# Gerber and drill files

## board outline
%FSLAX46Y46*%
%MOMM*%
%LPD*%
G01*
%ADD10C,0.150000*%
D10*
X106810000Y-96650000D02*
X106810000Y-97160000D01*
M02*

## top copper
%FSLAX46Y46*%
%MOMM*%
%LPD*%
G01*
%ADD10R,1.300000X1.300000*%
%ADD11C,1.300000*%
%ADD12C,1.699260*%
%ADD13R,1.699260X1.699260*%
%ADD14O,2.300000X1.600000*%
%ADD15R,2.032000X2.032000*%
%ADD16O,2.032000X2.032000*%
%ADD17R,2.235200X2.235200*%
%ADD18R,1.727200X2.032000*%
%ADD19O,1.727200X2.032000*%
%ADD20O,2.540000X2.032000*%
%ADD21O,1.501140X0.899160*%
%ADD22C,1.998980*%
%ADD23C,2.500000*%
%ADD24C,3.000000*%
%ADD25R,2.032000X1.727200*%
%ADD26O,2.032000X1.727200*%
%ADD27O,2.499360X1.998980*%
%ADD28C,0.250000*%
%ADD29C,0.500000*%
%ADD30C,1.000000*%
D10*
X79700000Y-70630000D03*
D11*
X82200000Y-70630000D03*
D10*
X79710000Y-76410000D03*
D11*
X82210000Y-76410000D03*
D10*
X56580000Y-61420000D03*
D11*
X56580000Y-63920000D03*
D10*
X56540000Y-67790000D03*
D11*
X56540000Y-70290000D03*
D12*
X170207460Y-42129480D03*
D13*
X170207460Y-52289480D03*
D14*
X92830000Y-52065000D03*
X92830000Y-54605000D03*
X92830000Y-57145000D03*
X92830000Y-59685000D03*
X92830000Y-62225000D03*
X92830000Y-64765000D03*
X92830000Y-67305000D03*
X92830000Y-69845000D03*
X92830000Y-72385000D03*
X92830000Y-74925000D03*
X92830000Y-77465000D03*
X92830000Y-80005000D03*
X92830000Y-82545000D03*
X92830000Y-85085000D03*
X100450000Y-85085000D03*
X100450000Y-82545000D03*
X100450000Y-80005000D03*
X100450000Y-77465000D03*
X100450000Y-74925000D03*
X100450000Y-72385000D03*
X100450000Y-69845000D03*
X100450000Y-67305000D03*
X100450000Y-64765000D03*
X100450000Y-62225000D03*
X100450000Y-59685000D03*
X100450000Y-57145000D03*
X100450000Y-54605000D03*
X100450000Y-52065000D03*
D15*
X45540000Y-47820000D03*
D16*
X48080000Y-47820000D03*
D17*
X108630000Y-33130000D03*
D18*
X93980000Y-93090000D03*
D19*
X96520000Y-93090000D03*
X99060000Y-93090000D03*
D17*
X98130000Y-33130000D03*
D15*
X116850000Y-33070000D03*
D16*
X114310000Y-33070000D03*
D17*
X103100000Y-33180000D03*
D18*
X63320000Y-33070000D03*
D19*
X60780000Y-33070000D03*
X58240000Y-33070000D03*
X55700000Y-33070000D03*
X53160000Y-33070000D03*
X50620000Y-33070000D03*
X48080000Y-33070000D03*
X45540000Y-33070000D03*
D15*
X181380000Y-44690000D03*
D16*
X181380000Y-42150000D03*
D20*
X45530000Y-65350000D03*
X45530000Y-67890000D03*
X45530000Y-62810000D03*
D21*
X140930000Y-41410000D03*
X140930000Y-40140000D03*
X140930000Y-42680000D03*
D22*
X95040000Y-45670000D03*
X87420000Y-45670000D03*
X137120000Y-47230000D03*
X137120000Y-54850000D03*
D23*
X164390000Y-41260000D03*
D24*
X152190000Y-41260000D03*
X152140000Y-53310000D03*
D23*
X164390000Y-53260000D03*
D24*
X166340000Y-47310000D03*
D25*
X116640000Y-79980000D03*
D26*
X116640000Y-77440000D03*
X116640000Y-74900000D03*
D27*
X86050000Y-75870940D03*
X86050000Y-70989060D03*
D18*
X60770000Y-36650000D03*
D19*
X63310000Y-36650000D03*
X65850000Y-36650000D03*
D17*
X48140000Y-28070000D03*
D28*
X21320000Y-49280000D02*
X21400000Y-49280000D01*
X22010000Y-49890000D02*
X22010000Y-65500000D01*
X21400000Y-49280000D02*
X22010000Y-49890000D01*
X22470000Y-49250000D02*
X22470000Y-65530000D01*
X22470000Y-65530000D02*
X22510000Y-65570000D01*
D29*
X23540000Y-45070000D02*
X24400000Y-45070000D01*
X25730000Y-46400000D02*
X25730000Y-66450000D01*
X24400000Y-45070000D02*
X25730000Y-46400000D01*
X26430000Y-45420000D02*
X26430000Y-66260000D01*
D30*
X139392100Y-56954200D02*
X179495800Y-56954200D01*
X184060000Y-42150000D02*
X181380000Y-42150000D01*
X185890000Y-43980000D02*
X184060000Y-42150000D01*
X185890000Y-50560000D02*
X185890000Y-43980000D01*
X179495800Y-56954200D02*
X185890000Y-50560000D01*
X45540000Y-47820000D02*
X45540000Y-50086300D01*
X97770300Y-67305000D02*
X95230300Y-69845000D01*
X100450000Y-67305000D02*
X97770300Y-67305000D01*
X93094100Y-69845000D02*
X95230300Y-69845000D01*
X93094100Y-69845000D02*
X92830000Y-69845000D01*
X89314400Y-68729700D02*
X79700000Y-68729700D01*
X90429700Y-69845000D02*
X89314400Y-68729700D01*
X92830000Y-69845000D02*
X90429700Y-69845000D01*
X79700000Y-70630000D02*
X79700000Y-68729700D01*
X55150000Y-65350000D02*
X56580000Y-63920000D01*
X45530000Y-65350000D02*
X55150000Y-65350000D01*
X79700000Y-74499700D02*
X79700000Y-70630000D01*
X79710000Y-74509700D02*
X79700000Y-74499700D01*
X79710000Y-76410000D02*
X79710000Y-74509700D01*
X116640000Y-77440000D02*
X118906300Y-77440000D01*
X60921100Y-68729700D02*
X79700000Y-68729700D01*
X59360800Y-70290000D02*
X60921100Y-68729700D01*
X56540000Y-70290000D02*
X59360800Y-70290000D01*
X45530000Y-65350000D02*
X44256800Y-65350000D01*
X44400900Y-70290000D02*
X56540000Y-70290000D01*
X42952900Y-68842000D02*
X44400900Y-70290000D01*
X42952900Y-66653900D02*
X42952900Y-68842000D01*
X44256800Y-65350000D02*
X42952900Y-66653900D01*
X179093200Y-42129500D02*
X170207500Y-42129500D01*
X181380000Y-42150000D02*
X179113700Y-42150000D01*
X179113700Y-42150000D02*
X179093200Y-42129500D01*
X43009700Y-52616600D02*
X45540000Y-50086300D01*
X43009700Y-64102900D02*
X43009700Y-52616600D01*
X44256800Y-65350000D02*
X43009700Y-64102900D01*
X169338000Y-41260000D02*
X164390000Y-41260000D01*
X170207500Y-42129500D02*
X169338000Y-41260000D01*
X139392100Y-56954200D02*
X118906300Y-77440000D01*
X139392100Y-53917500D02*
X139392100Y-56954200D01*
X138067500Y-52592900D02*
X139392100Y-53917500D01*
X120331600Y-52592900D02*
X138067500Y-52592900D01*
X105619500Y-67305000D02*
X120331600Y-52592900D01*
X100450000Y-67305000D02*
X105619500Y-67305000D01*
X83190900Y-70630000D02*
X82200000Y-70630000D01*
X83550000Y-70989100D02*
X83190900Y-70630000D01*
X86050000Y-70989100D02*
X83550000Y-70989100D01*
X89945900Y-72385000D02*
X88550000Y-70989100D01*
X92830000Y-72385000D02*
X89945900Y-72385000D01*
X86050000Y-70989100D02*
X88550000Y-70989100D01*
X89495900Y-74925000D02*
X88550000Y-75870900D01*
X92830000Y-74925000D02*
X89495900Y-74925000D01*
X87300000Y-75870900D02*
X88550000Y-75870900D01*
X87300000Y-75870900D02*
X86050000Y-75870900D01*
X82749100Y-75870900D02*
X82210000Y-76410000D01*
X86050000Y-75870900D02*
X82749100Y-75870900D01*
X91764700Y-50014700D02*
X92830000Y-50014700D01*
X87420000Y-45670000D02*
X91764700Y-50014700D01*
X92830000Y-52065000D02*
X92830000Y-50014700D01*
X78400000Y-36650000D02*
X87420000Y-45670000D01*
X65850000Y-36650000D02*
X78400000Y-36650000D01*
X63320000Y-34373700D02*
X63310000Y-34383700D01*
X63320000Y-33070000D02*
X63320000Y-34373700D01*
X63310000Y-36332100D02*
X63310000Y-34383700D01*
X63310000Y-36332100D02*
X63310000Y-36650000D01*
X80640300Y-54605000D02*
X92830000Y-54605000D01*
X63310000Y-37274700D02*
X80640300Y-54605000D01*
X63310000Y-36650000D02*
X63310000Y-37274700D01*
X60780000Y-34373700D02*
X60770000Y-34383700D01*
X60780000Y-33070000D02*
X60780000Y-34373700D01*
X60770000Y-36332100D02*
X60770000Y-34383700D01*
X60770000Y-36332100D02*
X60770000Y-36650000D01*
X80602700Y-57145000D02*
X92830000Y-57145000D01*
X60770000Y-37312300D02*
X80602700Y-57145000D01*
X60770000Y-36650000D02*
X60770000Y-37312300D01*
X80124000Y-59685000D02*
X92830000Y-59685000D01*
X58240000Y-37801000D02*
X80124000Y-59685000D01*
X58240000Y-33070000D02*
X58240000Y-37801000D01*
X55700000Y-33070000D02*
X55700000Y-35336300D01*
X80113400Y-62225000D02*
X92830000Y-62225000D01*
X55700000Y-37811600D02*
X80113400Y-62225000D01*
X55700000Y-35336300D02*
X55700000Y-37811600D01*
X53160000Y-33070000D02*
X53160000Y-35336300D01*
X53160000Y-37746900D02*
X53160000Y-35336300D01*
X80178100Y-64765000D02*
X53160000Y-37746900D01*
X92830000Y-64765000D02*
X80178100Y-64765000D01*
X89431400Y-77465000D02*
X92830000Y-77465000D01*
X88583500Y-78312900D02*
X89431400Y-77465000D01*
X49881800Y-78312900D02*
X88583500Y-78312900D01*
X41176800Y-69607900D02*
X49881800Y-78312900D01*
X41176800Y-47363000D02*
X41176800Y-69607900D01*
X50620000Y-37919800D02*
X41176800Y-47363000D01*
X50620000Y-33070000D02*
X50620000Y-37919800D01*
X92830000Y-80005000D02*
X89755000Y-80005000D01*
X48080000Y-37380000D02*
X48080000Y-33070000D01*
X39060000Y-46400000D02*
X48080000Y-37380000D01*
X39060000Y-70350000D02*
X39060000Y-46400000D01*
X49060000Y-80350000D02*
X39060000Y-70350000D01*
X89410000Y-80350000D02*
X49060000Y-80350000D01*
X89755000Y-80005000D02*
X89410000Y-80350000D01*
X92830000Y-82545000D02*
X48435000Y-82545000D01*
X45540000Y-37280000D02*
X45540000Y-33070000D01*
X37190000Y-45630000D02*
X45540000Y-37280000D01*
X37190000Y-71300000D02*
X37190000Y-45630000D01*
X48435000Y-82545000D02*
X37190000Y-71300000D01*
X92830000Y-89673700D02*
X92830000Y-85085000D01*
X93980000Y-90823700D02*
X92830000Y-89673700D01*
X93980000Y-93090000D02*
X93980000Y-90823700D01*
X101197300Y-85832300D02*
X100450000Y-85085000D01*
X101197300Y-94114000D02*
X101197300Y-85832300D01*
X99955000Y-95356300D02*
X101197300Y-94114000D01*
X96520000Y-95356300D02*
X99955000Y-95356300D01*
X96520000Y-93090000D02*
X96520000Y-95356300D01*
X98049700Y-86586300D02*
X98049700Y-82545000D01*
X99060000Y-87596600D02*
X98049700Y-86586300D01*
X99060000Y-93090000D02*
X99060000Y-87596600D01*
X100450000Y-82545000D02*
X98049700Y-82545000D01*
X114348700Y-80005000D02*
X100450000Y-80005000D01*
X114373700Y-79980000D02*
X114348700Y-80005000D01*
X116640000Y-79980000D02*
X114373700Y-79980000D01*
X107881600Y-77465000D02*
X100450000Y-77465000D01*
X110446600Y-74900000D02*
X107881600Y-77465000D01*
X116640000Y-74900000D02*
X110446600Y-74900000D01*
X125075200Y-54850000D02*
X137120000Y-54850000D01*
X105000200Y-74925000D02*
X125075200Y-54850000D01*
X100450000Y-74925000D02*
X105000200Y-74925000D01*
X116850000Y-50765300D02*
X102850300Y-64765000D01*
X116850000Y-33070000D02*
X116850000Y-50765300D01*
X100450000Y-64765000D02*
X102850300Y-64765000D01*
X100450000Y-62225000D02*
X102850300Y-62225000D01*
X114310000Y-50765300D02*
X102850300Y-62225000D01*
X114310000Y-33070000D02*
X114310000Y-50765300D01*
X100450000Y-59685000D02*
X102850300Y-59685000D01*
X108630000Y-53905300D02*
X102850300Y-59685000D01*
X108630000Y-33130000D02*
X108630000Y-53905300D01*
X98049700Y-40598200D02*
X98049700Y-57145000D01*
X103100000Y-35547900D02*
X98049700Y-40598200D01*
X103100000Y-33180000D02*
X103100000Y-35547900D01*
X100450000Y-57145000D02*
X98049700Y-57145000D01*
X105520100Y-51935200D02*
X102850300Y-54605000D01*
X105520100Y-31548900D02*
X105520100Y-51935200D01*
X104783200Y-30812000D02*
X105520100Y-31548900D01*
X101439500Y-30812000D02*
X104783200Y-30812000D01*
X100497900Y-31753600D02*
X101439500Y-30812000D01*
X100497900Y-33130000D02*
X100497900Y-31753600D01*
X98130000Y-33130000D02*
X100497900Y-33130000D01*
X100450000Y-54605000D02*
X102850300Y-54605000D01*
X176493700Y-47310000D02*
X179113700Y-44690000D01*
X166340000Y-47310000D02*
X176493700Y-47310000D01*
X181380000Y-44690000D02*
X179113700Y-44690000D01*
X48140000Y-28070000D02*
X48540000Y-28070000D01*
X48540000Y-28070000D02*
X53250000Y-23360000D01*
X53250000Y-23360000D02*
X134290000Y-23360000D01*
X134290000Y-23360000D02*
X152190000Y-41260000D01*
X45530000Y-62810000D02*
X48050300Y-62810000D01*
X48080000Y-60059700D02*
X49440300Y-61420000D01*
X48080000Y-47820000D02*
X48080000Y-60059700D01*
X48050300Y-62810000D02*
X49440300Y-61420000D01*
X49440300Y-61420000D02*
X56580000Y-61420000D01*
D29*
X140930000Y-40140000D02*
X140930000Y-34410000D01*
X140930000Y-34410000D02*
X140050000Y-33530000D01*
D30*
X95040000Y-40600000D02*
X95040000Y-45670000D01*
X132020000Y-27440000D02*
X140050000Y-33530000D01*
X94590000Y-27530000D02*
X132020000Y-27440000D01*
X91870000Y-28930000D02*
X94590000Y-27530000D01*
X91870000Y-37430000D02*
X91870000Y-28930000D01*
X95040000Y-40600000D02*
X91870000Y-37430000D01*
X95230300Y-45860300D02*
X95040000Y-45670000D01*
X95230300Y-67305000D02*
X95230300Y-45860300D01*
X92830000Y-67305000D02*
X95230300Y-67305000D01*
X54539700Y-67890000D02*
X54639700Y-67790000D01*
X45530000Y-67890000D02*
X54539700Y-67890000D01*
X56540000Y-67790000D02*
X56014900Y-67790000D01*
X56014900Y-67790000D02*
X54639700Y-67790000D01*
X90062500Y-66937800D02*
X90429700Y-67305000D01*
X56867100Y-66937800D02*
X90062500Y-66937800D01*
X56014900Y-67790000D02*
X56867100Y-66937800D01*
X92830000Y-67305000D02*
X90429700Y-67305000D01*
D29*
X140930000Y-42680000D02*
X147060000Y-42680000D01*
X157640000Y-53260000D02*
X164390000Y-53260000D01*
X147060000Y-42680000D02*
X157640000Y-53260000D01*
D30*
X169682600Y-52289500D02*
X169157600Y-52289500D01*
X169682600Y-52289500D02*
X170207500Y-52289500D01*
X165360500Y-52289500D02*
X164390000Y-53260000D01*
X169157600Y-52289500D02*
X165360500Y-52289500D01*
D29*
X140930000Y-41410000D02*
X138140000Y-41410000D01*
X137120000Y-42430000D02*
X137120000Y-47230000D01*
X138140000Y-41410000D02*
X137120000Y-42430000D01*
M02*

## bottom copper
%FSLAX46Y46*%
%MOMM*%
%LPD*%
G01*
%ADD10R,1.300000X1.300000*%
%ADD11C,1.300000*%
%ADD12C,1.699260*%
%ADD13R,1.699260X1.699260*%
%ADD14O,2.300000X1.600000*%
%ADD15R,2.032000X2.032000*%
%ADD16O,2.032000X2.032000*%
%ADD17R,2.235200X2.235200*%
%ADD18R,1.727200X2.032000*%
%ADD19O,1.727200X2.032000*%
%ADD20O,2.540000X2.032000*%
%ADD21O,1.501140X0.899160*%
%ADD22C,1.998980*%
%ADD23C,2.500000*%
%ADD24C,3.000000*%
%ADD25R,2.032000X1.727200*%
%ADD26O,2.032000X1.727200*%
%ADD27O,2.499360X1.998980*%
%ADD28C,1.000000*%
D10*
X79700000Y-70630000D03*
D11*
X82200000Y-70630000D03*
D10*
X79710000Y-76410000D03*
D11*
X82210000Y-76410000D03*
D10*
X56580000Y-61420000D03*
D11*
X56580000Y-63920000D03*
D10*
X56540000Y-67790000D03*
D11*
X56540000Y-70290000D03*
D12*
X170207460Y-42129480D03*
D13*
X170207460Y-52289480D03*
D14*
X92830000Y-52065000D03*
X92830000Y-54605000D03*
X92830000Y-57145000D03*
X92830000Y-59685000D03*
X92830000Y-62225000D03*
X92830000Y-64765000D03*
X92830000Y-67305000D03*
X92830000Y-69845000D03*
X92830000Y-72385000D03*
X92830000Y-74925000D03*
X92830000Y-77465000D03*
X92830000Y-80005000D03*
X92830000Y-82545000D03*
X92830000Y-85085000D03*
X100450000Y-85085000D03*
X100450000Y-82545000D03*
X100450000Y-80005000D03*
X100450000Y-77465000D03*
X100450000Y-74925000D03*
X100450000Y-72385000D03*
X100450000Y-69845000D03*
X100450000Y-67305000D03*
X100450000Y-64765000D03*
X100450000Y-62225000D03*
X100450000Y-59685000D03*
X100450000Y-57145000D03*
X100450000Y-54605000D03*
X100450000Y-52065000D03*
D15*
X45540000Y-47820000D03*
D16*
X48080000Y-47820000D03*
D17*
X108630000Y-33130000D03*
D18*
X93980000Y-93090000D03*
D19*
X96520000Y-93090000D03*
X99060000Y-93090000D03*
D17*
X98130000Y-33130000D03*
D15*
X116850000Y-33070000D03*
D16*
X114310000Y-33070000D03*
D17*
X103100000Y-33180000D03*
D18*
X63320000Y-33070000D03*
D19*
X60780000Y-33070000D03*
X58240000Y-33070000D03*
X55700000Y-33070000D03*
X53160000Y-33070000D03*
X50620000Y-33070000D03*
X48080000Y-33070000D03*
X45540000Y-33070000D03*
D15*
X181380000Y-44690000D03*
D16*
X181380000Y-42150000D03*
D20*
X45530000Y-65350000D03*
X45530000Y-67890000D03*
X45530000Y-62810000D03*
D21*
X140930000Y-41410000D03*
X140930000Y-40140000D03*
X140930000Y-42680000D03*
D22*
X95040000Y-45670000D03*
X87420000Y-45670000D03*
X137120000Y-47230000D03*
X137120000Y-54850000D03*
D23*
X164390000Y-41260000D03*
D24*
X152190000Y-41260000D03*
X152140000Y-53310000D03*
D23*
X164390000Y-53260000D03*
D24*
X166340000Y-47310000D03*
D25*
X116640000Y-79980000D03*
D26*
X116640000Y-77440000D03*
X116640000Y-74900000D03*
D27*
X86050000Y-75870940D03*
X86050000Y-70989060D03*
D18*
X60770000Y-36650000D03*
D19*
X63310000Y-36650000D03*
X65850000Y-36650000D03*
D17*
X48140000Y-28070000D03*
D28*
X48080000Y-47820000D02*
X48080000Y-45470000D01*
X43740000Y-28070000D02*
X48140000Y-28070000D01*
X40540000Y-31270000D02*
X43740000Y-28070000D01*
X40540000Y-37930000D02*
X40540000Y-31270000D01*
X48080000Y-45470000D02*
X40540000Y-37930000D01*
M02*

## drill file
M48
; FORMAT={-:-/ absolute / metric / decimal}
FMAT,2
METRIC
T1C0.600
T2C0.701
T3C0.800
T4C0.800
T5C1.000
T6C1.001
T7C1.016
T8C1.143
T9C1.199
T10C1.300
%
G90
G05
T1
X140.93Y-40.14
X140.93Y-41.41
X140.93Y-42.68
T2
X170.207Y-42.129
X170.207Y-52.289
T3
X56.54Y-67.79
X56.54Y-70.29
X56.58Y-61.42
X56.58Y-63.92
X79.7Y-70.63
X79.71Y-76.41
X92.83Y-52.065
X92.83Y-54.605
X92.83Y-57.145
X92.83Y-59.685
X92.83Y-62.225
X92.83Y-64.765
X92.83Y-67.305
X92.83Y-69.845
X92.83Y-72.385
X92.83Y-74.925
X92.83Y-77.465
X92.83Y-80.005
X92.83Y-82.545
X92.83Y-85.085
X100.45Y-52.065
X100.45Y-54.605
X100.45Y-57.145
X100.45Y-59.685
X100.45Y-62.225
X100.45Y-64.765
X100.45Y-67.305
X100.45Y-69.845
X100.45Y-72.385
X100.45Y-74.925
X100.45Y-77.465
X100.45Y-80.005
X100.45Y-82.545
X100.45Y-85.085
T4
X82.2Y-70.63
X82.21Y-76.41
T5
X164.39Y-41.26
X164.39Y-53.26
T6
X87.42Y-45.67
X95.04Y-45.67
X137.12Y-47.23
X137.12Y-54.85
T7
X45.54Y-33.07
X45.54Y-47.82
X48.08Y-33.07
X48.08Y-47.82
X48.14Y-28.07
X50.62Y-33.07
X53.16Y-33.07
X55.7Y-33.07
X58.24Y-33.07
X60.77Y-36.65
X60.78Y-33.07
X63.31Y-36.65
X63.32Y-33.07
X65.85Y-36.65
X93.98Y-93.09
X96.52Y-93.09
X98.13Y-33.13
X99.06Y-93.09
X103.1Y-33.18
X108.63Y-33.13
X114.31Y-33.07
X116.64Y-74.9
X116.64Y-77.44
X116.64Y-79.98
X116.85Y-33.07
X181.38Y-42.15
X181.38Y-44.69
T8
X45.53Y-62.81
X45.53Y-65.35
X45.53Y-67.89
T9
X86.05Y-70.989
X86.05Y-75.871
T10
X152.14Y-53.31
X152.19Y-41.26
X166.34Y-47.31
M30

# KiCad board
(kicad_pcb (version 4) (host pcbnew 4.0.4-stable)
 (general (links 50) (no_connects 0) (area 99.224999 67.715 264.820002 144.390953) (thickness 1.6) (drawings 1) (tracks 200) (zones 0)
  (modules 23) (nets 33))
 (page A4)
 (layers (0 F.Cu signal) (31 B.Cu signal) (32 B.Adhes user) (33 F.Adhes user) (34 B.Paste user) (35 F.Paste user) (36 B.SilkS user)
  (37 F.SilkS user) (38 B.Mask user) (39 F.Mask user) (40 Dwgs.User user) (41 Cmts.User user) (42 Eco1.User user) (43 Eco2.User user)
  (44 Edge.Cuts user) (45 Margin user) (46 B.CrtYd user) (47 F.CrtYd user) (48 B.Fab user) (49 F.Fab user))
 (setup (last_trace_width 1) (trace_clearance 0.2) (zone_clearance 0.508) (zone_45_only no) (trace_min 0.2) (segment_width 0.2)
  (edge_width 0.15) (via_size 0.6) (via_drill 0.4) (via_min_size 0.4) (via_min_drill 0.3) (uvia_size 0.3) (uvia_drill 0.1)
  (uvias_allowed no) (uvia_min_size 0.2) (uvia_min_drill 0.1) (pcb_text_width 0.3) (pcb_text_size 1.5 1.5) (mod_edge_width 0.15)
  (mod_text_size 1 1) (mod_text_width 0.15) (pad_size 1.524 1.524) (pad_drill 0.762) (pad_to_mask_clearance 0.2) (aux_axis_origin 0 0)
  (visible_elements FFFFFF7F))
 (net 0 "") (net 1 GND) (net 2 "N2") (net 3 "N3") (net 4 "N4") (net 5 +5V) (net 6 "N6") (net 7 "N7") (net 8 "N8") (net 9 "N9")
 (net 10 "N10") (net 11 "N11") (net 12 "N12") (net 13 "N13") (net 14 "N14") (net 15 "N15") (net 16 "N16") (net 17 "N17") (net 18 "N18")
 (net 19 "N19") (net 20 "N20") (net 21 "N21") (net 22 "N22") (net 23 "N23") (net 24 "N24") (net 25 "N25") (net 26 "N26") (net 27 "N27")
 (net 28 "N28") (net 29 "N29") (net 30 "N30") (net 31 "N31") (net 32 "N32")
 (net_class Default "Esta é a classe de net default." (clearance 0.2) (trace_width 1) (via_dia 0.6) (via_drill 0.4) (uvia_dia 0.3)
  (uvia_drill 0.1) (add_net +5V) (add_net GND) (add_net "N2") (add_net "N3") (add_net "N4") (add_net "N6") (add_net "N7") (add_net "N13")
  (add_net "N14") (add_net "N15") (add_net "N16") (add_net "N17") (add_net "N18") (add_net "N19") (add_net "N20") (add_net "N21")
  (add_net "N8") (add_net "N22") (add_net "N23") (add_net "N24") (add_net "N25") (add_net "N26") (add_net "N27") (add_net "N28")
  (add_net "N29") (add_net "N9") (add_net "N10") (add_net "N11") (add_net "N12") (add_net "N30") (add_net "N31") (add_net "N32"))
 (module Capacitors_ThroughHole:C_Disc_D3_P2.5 (layer F.Cu) (at 79.7 70.63)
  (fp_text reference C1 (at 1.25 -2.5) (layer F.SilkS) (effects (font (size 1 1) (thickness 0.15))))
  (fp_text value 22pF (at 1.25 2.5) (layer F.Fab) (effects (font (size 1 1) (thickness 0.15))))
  (pad 1 thru_hole rect (at 0 0) (size 1.3 1.3) (drill 0.8) (layers *.Cu *.Mask F.SilkS) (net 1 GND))
  (pad 2 thru_hole circle (at 2.5 0) (size 1.3 1.3) (drill 0.8001) (layers *.Cu *.Mask F.SilkS) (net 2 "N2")))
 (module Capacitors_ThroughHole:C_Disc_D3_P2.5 (layer F.Cu) (at 79.71 76.41)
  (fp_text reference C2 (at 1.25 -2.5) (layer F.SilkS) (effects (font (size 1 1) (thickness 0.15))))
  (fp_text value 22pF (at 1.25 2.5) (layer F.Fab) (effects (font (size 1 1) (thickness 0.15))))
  (pad 1 thru_hole rect (at 0 0) (size 1.3 1.3) (drill 0.8) (layers *.Cu *.Mask F.SilkS) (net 1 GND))
  (pad 2 thru_hole circle (at 2.5 0) (size 1.3 1.3) (drill 0.8001) (layers *.Cu *.Mask F.SilkS) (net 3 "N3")))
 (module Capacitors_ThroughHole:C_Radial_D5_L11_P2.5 (layer F.Cu) (at 56.58 61.42 270)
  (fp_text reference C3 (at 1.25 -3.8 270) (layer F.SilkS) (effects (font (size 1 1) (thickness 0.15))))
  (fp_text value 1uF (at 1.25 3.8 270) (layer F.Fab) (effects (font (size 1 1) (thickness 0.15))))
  (pad 1 thru_hole rect (at 0 0 270) (size 1.3 1.3) (drill 0.8) (layers *.Cu *.Mask F.SilkS) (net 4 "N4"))
  (pad 2 thru_hole circle (at 2.5 0 270) (size 1.3 1.3) (drill 0.8) (layers *.Cu *.Mask F.SilkS) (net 1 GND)))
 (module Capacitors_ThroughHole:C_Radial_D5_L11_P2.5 (layer F.Cu) (at 56.54 67.79 270)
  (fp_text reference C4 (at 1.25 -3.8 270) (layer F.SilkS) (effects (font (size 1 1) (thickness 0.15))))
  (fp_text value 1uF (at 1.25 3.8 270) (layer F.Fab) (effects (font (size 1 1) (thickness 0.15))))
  (pad 1 thru_hole rect (at 0 0 270) (size 1.3 1.3) (drill 0.8) (layers *.Cu *.Mask F.SilkS) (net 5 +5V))
  (pad 2 thru_hole circle (at 2.5 0 270) (size 1.3 1.3) (drill 0.8) (layers *.Cu *.Mask F.SilkS) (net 1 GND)))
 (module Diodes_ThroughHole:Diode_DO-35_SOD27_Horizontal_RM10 (layer F.Cu) (at 170.21 52.29 90)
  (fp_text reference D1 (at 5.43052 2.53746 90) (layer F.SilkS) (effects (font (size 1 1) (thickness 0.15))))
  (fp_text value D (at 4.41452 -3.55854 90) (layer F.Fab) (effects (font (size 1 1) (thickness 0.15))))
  (pad 2 thru_hole circle (at 10.16052 -0.00254 270) (size 1.69926 1.69926) (drill 0.70104) (layers *.Cu *.Mask F.SilkS) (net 1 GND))
  (pad 1 thru_hole rect (at 0.00052 -0.00254 270) (size 1.69926 1.69926) (drill 0.70104) (layers *.Cu *.Mask F.SilkS) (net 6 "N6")))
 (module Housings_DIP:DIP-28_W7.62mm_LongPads (layer F.Cu) (at 92.83 52.065)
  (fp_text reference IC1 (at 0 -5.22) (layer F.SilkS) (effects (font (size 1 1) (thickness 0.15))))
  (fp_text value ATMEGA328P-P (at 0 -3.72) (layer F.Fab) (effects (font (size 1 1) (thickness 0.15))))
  (pad 1 thru_hole oval (at 0 0) (size 2.3 1.6) (drill 0.8) (layers *.Cu *.Mask F.SilkS) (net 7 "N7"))
  (pad 2 thru_hole oval (at 0 2.54) (size 2.3 1.6) (drill 0.8) (layers *.Cu *.Mask F.SilkS) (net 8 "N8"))
  (pad 3 thru_hole oval (at 0 5.08) (size 2.3 1.6) (drill 0.8) (layers *.Cu *.Mask F.SilkS) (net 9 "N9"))
  (pad 4 thru_hole oval (at 0 7.62) (size 2.3 1.6) (drill 0.8) (layers *.Cu *.Mask F.SilkS) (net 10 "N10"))
  (pad 5 thru_hole oval (at 0 10.16) (size 2.3 1.6) (drill 0.8) (layers *.Cu *.Mask F.SilkS) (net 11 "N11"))
  (pad 6 thru_hole oval (at 0 12.7) (size 2.3 1.6) (drill 0.8) (layers *.Cu *.Mask F.SilkS) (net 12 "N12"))
  (pad 7 thru_hole oval (at 0 15.24) (size 2.3 1.6) (drill 0.8) (layers *.Cu *.Mask F.SilkS) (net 5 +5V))
  (pad 8 thru_hole oval (at 0 17.78) (size 2.3 1.6) (drill 0.8) (layers *.Cu *.Mask F.SilkS) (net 1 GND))
  (pad 9 thru_hole oval (at 0 20.32) (size 2.3 1.6) (drill 0.8) (layers *.Cu *.Mask F.SilkS) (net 2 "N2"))
  (pad 10 thru_hole oval (at 0 22.86) (size 2.3 1.6) (drill 0.8) (layers *.Cu *.Mask F.SilkS) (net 3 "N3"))
  (pad 11 thru_hole oval (at 0 25.4) (size 2.3 1.6) (drill 0.8) (layers *.Cu *.Mask F.SilkS) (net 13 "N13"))
  (pad 12 thru_hole oval (at 0 27.94) (size 2.3 1.6) (drill 0.8) (layers *.Cu *.Mask F.SilkS) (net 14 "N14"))
  (pad 13 thru_hole oval (at 0 30.48) (size 2.3 1.6) (drill 0.8) (layers *.Cu *.Mask F.SilkS) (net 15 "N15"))
  (pad 14 thru_hole oval (at 0 33.02) (size 2.3 1.6) (drill 0.8) (layers *.Cu *.Mask F.SilkS) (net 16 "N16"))
  (pad 15 thru_hole oval (at 7.62 33.02) (size 2.3 1.6) (drill 0.8) (layers *.Cu *.Mask F.SilkS) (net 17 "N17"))
  (pad 16 thru_hole oval (at 7.62 30.48) (size 2.3 1.6) (drill 0.8) (layers *.Cu *.Mask F.SilkS) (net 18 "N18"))
  (pad 17 thru_hole oval (at 7.62 27.94) (size 2.3 1.6) (drill 0.8) (layers *.Cu *.Mask F.SilkS) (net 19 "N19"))
  (pad 18 thru_hole oval (at 7.62 25.4) (size 2.3 1.6) (drill 0.8) (layers *.Cu *.Mask F.SilkS) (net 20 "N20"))
  (pad 19 thru_hole oval (at 7.62 22.86) (size 2.3 1.6) (drill 0.8) (layers *.Cu *.Mask F.SilkS) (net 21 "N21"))
  (pad 20 thru_hole oval (at 7.62 20.32) (size 2.3 1.6) (drill 0.8) (layers *.Cu *.Mask F.SilkS) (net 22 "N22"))
  (pad 21 thru_hole oval (at 7.62 17.78) (size 2.3 1.6) (drill 0.8) (layers *.Cu *.Mask F.SilkS) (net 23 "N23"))
  (pad 22 thru_hole oval (at 7.62 15.24) (size 2.3 1.6) (drill 0.8) (layers *.Cu *.Mask F.SilkS) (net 1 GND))
  (pad 23 thru_hole oval (at 7.62 12.7) (size 2.3 1.6) (drill 0.8) (layers *.Cu *.Mask F.SilkS) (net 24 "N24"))
  (pad 24 thru_hole oval (at 7.62 10.16) (size 2.3 1.6) (drill 0.8) (layers *.Cu *.Mask F.SilkS) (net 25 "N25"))
  (pad 25 thru_hole oval (at 7.62 7.62) (size 2.3 1.6) (drill 0.8) (layers *.Cu *.Mask F.SilkS) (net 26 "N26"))
  (pad 26 thru_hole oval (at 7.62 5.08) (size 2.3 1.6) (drill 0.8) (layers *.Cu *.Mask F.SilkS) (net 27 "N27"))
  (pad 27 thru_hole oval (at 7.62 2.54) (size 2.3 1.6) (drill 0.8) (layers *.Cu *.Mask F.SilkS) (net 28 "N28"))
  (pad 28 thru_hole oval (at 7.62 0) (size 2.3 1.6) (drill 0.8) (layers *.Cu *.Mask F.SilkS) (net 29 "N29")))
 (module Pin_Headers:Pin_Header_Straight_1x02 (layer F.Cu) (at 45.54 47.82 90)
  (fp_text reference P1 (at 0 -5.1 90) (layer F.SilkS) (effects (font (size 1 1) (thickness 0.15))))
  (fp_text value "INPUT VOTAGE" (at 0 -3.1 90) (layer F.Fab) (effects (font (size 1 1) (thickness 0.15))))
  (pad 1 thru_hole rect (at 0 0 90) (size 2.032 2.032) (drill 1.016) (layers *.Cu *.Mask F.SilkS) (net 1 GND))
  (pad 2 thru_hole oval (at 0 2.54 90) (size 2.032 2.032) (drill 1.016) (layers *.Cu *.Mask F.SilkS) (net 4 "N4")))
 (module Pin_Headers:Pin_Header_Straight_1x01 (layer F.Cu) (at 108.63 33.13)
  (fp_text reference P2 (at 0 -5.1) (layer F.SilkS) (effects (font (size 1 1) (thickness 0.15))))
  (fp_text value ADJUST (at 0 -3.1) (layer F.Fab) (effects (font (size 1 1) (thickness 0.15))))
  (pad 1 thru_hole rect (at 0 0) (size 2.2352 2.2352) (drill 1.016) (layers *.Cu *.Mask F.SilkS) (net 26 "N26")))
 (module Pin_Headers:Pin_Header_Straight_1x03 (layer F.Cu) (at 93.98 93.09 90)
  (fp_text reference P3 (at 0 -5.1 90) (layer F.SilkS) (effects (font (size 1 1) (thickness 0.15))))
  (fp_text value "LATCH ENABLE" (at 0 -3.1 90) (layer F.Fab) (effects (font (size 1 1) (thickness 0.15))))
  (pad 1 thru_hole rect (at 0 0 90) (size 2.032 1.7272) (drill 1.016) (layers *.Cu *.Mask F.SilkS) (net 16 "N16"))
  (pad 2 thru_hole oval (at 0 2.54 90) (size 2.032 1.7272) (drill 1.016) (layers *.Cu *.Mask F.SilkS) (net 17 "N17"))
  (pad 3 thru_hole oval (at 0 5.08 90) (size 2.032 1.7272) (drill 1.016) (layers *.Cu *.Mask F.SilkS) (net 18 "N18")))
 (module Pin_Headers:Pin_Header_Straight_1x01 (layer F.Cu) (at 98.13 33.13)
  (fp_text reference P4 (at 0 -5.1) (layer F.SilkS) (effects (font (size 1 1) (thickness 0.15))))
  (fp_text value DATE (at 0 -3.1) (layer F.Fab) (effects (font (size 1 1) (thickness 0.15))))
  (pad 1 thru_hole rect (at 0 0) (size 2.2352 2.2352) (drill 1.016) (layers *.Cu *.Mask F.SilkS) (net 28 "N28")))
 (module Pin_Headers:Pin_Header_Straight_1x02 (layer F.Cu) (at 116.85 33.07 270)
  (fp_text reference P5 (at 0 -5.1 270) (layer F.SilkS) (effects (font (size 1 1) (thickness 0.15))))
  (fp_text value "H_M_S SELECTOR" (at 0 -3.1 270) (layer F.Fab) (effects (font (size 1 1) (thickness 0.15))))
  (pad 1 thru_hole rect (at 0 0 270) (size 2.032 2.032) (drill 1.016) (layers *.Cu *.Mask F.SilkS) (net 24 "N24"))
  (pad 2 thru_hole oval (at 0 2.54 270) (size 2.032 2.032) (drill 1.016) (layers *.Cu *.Mask F.SilkS) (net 25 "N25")))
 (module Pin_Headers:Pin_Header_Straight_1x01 (layer F.Cu) (at 103.1 33.18)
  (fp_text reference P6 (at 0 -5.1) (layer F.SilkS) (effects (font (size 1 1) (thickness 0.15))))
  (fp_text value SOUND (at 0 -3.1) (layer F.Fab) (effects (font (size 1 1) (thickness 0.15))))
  (pad 1 thru_hole rect (at 0 0) (size 2.2352 2.2352) (drill 1.016) (layers *.Cu *.Mask F.SilkS) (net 27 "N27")))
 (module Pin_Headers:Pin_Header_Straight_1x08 (layer F.Cu) (at 63.32 33.07 270)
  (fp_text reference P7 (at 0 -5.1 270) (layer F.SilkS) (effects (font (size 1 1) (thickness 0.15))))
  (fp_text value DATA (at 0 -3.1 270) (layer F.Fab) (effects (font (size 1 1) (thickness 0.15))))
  (pad 1 thru_hole rect (at 0 0 270) (size 2.032 1.7272) (drill 1.016) (layers *.Cu *.Mask F.SilkS) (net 8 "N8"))
  (pad 2 thru_hole oval (at 0 2.54 270) (size 2.032 1.7272) (drill 1.016) (layers *.Cu *.Mask F.SilkS) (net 9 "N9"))
  (pad 3 thru_hole oval (at 0 5.08 270) (size 2.032 1.7272) (drill 1.016) (layers *.Cu *.Mask F.SilkS) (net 10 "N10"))
  (pad 4 thru_hole oval (at 0 7.62 270) (size 2.032 1.7272) (drill 1.016) (layers *.Cu *.Mask F.SilkS) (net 11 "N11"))
  (pad 5 thru_hole oval (at 0 10.16 270) (size 2.032 1.7272) (drill 1.016) (layers *.Cu *.Mask F.SilkS) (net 12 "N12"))
  (pad 6 thru_hole oval (at 0 12.7 270) (size 2.032 1.7272) (drill 1.016) (layers *.Cu *.Mask F.SilkS) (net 13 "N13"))
  (pad 7 thru_hole oval (at 0 15.24 270) (size 2.032 1.7272) (drill 1.016) (layers *.Cu *.Mask F.SilkS) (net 14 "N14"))
  (pad 8 thru_hole oval (at 0 17.78 270) (size 2.032 1.7272) (drill 1.016) (layers *.Cu *.Mask F.SilkS) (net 15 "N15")))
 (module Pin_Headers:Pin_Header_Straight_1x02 (layer F.Cu) (at 181.38 44.69 180)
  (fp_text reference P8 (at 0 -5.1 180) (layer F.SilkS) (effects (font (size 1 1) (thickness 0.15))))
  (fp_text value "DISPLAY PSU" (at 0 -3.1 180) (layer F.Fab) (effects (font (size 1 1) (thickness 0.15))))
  (pad 1 thru_hole rect (at 0 0 180) (size 2.032 2.032) (drill 1.016) (layers *.Cu *.Mask F.SilkS) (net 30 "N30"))
  (pad 2 thru_hole oval (at 0 2.54 180) (size 2.032 2.032) (drill 1.016) (layers *.Cu *.Mask F.SilkS) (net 1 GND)))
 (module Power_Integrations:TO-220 (layer F.Cu) (at 45.53 65.35 270)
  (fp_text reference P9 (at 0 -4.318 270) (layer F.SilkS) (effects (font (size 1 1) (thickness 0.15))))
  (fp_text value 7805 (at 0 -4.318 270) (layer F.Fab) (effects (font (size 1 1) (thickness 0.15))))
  (pad 2 thru_hole oval (at 0 0 270) (size 2.032 2.54) (drill 1.143) (layers *.Cu *.Mask F.SilkS) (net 1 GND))
  (pad 3 thru_hole oval (at 2.54 0 270) (size 2.032 2.54) (drill 1.143) (layers *.Cu *.Mask F.SilkS) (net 5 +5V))
  (pad 1 thru_hole oval (at -2.54 0 270) (size 2.032 2.54) (drill 1.143) (layers *.Cu *.Mask F.SilkS) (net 4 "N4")))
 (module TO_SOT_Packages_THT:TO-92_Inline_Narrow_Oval (layer F.Cu) (at 140.93 42.68 90)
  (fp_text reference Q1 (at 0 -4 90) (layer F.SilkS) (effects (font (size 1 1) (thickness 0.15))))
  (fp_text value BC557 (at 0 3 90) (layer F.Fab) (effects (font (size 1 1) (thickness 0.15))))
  (pad 2 thru_hole oval (at 1.27 0 270) (size 0.89916 1.50114) (drill 0.6) (layers *.Cu *.Mask F.SilkS) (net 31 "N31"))
  (pad 3 thru_hole oval (at 2.54 0 270) (size 0.89916 1.50114) (drill 0.6) (layers *.Cu *.Mask F.SilkS) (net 5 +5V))
  (pad 1 thru_hole oval (at 0 0 270) (size 0.89916 1.50114) (drill 0.6) (layers *.Cu *.Mask F.SilkS) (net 6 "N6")))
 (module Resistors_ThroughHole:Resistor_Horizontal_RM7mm (layer F.Cu) (at 95.04 45.67 180)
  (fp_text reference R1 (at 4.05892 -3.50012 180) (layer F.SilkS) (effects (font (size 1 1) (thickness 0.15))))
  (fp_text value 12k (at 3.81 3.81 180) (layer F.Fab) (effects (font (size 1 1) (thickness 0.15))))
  (pad 1 thru_hole circle (at 0 0 180) (size 1.99898 1.99898) (drill 1.00076) (layers *.Cu *.SilkS *.Mask) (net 5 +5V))
  (pad 2 thru_hole circle (at 7.62 0 180) (size 1.99898 1.99898) (drill 1.00076) (layers *.Cu *.SilkS *.Mask) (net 7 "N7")))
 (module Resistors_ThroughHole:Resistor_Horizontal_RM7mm (layer F.Cu) (at 137.12 47.23 270)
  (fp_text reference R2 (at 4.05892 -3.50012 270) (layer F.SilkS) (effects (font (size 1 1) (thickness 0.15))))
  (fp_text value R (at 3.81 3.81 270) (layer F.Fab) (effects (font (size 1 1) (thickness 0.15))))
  (pad 1 thru_hole circle (at 0 0 270) (size 1.99898 1.99898) (drill 1.00076) (layers *.Cu *.SilkS *.Mask) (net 31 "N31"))
  (pad 2 thru_hole circle (at 7.62 0 270) (size 1.99898 1.99898) (drill 1.00076) (layers *.Cu *.SilkS *.Mask) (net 21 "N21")))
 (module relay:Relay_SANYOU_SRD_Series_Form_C (layer F.Cu) (at 166.34 47.31 180)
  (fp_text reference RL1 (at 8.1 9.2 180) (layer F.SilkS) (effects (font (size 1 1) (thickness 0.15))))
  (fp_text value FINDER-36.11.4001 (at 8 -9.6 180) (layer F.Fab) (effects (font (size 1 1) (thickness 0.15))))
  (pad 2 thru_hole circle (at 1.95 6.05 270) (size 2.5 2.5) (drill 1) (layers *.Cu *.Mask) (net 1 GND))
  (pad 3 thru_hole circle (at 14.15 6.05 270) (size 3 3) (drill 1.3) (layers *.Cu *.Mask) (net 4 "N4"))
  (pad 4 thru_hole circle (at 14.2 -6 270) (size 3 3) (drill 1.3) (layers *.Cu *.Mask) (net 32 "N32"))
  (pad 5 thru_hole circle (at 1.95 -5.95 270) (size 2.5 2.5) (drill 1) (layers *.Cu *.Mask F.SilkS) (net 6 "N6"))
  (pad 1 thru_hole circle (at 0 0 270) (size 3 3) (drill 1.3) (layers *.Cu *.Mask) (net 30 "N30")))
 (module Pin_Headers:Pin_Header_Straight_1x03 (layer F.Cu) (at 116.64 79.98 180)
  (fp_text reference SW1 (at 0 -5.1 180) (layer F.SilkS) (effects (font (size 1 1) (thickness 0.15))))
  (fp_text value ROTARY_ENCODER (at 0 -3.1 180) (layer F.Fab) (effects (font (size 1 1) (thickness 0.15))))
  (pad 1 thru_hole rect (at 0 0 180) (size 2.032 1.7272) (drill 1.016) (layers *.Cu *.Mask F.SilkS) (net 19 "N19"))
  (pad 2 thru_hole oval (at 0 2.54 180) (size 2.032 1.7272) (drill 1.016) (layers *.Cu *.Mask F.SilkS) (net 1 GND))
  (pad 3 thru_hole oval (at 0 5.08 180) (size 2.032 1.7272) (drill 1.016) (layers *.Cu *.Mask F.SilkS) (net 20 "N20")))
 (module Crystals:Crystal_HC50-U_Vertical (layer F.Cu) (at 86.05 73.43 90)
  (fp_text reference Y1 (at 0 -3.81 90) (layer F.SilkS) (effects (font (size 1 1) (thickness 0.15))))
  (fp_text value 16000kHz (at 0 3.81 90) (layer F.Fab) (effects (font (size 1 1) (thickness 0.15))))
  (pad 1 thru_hole oval (at -2.44094 0 90) (size 1.99898 2.49936) (drill 1.19888) (layers *.Cu *.Mask F.SilkS) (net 3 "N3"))
  (pad 2 thru_hole oval (at 2.44094 0 90) (size 1.99898 2.49936) (drill 1.19888) (layers *.Cu *.Mask F.SilkS) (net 2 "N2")))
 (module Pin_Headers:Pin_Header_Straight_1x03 (layer F.Cu) (at 60.77 36.65 90)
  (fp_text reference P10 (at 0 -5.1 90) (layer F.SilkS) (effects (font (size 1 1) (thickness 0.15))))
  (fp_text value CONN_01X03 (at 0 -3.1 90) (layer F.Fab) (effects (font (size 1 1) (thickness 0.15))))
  (pad 1 thru_hole rect (at 0 0 90) (size 2.032 1.7272) (drill 1.016) (layers *.Cu *.Mask F.SilkS) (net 9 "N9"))
  (pad 2 thru_hole oval (at 0 2.54 90) (size 2.032 1.7272) (drill 1.016) (layers *.Cu *.Mask F.SilkS) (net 8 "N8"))
  (pad 3 thru_hole oval (at 0 5.08 90) (size 2.032 1.7272) (drill 1.016) (layers *.Cu *.Mask F.SilkS) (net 7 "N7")))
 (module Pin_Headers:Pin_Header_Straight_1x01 (layer F.Cu) (at 48.14 28.07)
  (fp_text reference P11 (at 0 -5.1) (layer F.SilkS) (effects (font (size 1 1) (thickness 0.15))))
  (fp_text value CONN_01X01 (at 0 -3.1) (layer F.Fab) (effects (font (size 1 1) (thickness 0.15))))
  (pad 1 thru_hole rect (at 0 0) (size 2.2352 2.2352) (drill 1.016) (layers *.Cu *.Mask) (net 4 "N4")))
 (gr_line (start 106.81 96.65) (end 106.81 97.16) (angle 90) (layer Edge.Cuts) (width 0.15))
 (segment (start 21.32 49.28) (end 21.4 49.28) (width 0.25) (layer F.Cu) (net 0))
 (segment (start 22.01 49.89) (end 22.01 65.5) (width 0.25) (layer F.Cu) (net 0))
 (segment (start 21.4 49.28) (end 22.01 49.89) (width 0.25) (layer F.Cu) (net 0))
 (segment (start 22.47 49.25) (end 22.47 65.53) (width 0.25) (layer F.Cu) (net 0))
 (segment (start 22.47 65.53) (end 22.51 65.57) (width 0.25) (layer F.Cu) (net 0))
 (segment (start 23.54 45.07) (end 24.4 45.07) (width 0.5) (layer F.Cu) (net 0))
 (segment (start 25.73 46.4) (end 25.73 66.45) (width 0.5) (layer F.Cu) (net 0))
 (segment (start 24.4 45.07) (end 25.73 46.4) (width 0.5) (layer F.Cu) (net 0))
 (segment (start 26.43 45.42) (end 26.43 66.26) (width 0.5) (layer F.Cu) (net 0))
 (segment (start 139.3921 56.9542) (end 179.4958 56.9542) (width 1) (layer F.Cu) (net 1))
 (segment (start 184.06 42.15) (end 181.38 42.15) (width 1) (layer F.Cu) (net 1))
 (segment (start 185.89 43.98) (end 184.06 42.15) (width 1) (layer F.Cu) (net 1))
 (segment (start 185.89 50.56) (end 185.89 43.98) (width 1) (layer F.Cu) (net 1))
 (segment (start 179.4958 56.9542) (end 185.89 50.56) (width 1) (layer F.Cu) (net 1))
 (segment (start 45.54 47.82) (end 45.54 50.0863) (width 1) (layer F.Cu) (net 1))
 (segment (start 97.7703 67.305) (end 95.2303 69.845) (width 1) (layer F.Cu) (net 1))
 (segment (start 100.45 67.305) (end 97.7703 67.305) (width 1) (layer F.Cu) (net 1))
 (segment (start 93.0941 69.845) (end 95.2303 69.845) (width 1) (layer F.Cu) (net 1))
 (segment (start 93.0941 69.845) (end 92.83 69.845) (width 1) (layer F.Cu) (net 1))
 (segment (start 89.3144 68.7297) (end 79.7 68.7297) (width 1) (layer F.Cu) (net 1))
 (segment (start 90.4297 69.845) (end 89.3144 68.7297) (width 1) (layer F.Cu) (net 1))
 (segment (start 92.83 69.845) (end 90.4297 69.845) (width 1) (layer F.Cu) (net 1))
 (segment (start 79.7 70.63) (end 79.7 68.7297) (width 1) (layer F.Cu) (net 1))
 (segment (start 55.15 65.35) (end 56.58 63.92) (width 1) (layer F.Cu) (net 1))
 (segment (start 45.53 65.35) (end 55.15 65.35) (width 1) (layer F.Cu) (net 1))
 (segment (start 79.7 74.4997) (end 79.7 70.63) (width 1) (layer F.Cu) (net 1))
 (segment (start 79.71 74.5097) (end 79.7 74.4997) (width 1) (layer F.Cu) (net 1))
 (segment (start 79.71 76.41) (end 79.71 74.5097) (width 1) (layer F.Cu) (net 1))
 (segment (start 116.64 77.44) (end 118.9063 77.44) (width 1) (layer F.Cu) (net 1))
 (segment (start 60.9211 68.7297) (end 79.7 68.7297) (width 1) (layer F.Cu) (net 1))
 (segment (start 59.3608 70.29) (end 60.9211 68.7297) (width 1) (layer F.Cu) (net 1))
 (segment (start 56.54 70.29) (end 59.3608 70.29) (width 1) (layer F.Cu) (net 1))
 (segment (start 45.53 65.35) (end 44.2568 65.35) (width 1) (layer F.Cu) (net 1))
 (segment (start 44.4009 70.29) (end 56.54 70.29) (width 1) (layer F.Cu) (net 1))
 (segment (start 42.9529 68.842) (end 44.4009 70.29) (width 1) (layer F.Cu) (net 1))
 (segment (start 42.9529 66.6539) (end 42.9529 68.842) (width 1) (layer F.Cu) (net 1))
 (segment (start 44.2568 65.35) (end 42.9529 66.6539) (width 1) (layer F.Cu) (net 1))
 (segment (start 179.0932 42.1295) (end 170.2075 42.1295) (width 1) (layer F.Cu) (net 1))
 (segment (start 181.38 42.15) (end 179.1137 42.15) (width 1) (layer F.Cu) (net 1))
 (segment (start 179.1137 42.15) (end 179.0932 42.1295) (width 1) (layer F.Cu) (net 1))
 (segment (start 43.0097 52.6166) (end 45.54 50.0863) (width 1) (layer F.Cu) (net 1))
 (segment (start 43.0097 64.1029) (end 43.0097 52.6166) (width 1) (layer F.Cu) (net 1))
 (segment (start 44.2568 65.35) (end 43.0097 64.1029) (width 1) (layer F.Cu) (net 1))
 (segment (start 169.338 41.26) (end 164.39 41.26) (width 1) (layer F.Cu) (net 1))
 (segment (start 170.2075 42.1295) (end 169.338 41.26) (width 1) (layer F.Cu) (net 1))
 (segment (start 139.3921 56.9542) (end 118.9063 77.44) (width 1) (layer F.Cu) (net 1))
 (segment (start 139.3921 53.9175) (end 139.3921 56.9542) (width 1) (layer F.Cu) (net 1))
 (segment (start 138.0675 52.5929) (end 139.3921 53.9175) (width 1) (layer F.Cu) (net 1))
 (segment (start 120.3316 52.5929) (end 138.0675 52.5929) (width 1) (layer F.Cu) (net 1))
 (segment (start 105.6195 67.305) (end 120.3316 52.5929) (width 1) (layer F.Cu) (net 1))
 (segment (start 100.45 67.305) (end 105.6195 67.305) (width 1) (layer F.Cu) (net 1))
 (segment (start 83.1909 70.63) (end 82.2 70.63) (width 1) (layer F.Cu) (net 2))
 (segment (start 83.55 70.9891) (end 83.1909 70.63) (width 1) (layer F.Cu) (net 2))
 (segment (start 86.05 70.9891) (end 83.55 70.9891) (width 1) (layer F.Cu) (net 2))
 (segment (start 89.9459 72.385) (end 88.55 70.9891) (width 1) (layer F.Cu) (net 2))
 (segment (start 92.83 72.385) (end 89.9459 72.385) (width 1) (layer F.Cu) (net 2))
 (segment (start 86.05 70.9891) (end 88.55 70.9891) (width 1) (layer F.Cu) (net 2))
 (segment (start 89.4959 74.925) (end 88.55 75.8709) (width 1) (layer F.Cu) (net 3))
 (segment (start 92.83 74.925) (end 89.4959 74.925) (width 1) (layer F.Cu) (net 3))
 (segment (start 87.3 75.8709) (end 88.55 75.8709) (width 1) (layer F.Cu) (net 3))
 (segment (start 87.3 75.8709) (end 86.05 75.8709) (width 1) (layer F.Cu) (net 3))
 (segment (start 82.7491 75.8709) (end 82.21 76.41) (width 1) (layer F.Cu) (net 3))
 (segment (start 86.05 75.8709) (end 82.7491 75.8709) (width 1) (layer F.Cu) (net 3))
 (segment (start 91.7647 50.0147) (end 92.83 50.0147) (width 1) (layer F.Cu) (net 7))
 (segment (start 87.42 45.67) (end 91.7647 50.0147) (width 1) (layer F.Cu) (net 7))
 (segment (start 92.83 52.065) (end 92.83 50.0147) (width 1) (layer F.Cu) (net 7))
 (segment (start 78.4 36.65) (end 87.42 45.67) (width 1) (layer F.Cu) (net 7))
 (segment (start 65.85 36.65) (end 78.4 36.65) (width 1) (layer F.Cu) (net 7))
 (segment (start 63.32 34.3737) (end 63.31 34.3837) (width 1) (layer F.Cu) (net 8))
 (segment (start 63.32 33.07) (end 63.32 34.3737) (width 1) (layer F.Cu) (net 8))
 (segment (start 63.31 36.3321) (end 63.31 34.3837) (width 1) (layer F.Cu) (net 8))
 (segment (start 63.31 36.3321) (end 63.31 36.65) (width 1) (layer F.Cu) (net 8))
 (segment (start 80.6403 54.605) (end 92.83 54.605) (width 1) (layer F.Cu) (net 8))
 (segment (start 63.31 37.2747) (end 80.6403 54.605) (width 1) (layer F.Cu) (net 8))
 (segment (start 63.31 36.65) (end 63.31 37.2747) (width 1) (layer F.Cu) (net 8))
 (segment (start 60.78 34.3737) (end 60.77 34.3837) (width 1) (layer F.Cu) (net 9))
 (segment (start 60.78 33.07) (end 60.78 34.3737) (width 1) (layer F.Cu) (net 9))
 (segment (start 60.77 36.3321) (end 60.77 34.3837) (width 1) (layer F.Cu) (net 9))
 (segment (start 60.77 36.3321) (end 60.77 36.65) (width 1) (layer F.Cu) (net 9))
 (segment (start 80.6027 57.145) (end 92.83 57.145) (width 1) (layer F.Cu) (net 9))
 (segment (start 60.77 37.3123) (end 80.6027 57.145) (width 1) (layer F.Cu) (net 9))
 (segment (start 60.77 36.65) (end 60.77 37.3123) (width 1) (layer F.Cu) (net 9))
 (segment (start 80.124 59.685) (end 92.83 59.685) (width 1) (layer F.Cu) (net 10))
 (segment (start 58.24 37.801) (end 80.124 59.685) (width 1) (layer F.Cu) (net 10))
 (segment (start 58.24 33.07) (end 58.24 37.801) (width 1) (layer F.Cu) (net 10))
 (segment (start 55.7 33.07) (end 55.7 35.3363) (width 1) (layer F.Cu) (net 11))
 (segment (start 80.1134 62.225) (end 92.83 62.225) (width 1) (layer F.Cu) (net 11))
 (segment (start 55.7 37.8116) (end 80.1134 62.225) (width 1) (layer F.Cu) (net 11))
 (segment (start 55.7 35.3363) (end 55.7 37.8116) (width 1) (layer F.Cu) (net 11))
 (segment (start 53.16 33.07) (end 53.16 35.3363) (width 1) (layer F.Cu) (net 12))
 (segment (start 53.16 37.7469) (end 53.16 35.3363) (width 1) (layer F.Cu) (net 12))
 (segment (start 80.1781 64.765) (end 53.16 37.7469) (width 1) (layer F.Cu) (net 12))
 (segment (start 92.83 64.765) (end 80.1781 64.765) (width 1) (layer F.Cu) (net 12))
 (segment (start 89.4314 77.465) (end 92.83 77.465) (width 1) (layer F.Cu) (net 13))
 (segment (start 88.5835 78.3129) (end 89.4314 77.465) (width 1) (layer F.Cu) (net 13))
 (segment (start 49.8818 78.3129) (end 88.5835 78.3129) (width 1) (layer F.Cu) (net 13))
 (segment (start 41.1768 69.6079) (end 49.8818 78.3129) (width 1) (layer F.Cu) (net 13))
 (segment (start 41.1768 47.363) (end 41.1768 69.6079) (width 1) (layer F.Cu) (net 13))
 (segment (start 50.62 37.9198) (end 41.1768 47.363) (width 1) (layer F.Cu) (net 13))
 (segment (start 50.62 33.07) (end 50.62 37.9198) (width 1) (layer F.Cu) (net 13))
 (segment (start 92.83 80.005) (end 89.755 80.005) (width 1) (layer F.Cu) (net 14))
 (segment (start 48.08 37.38) (end 48.08 33.07) (width 1) (layer F.Cu) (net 14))
 (segment (start 39.06 46.4) (end 48.08 37.38) (width 1) (layer F.Cu) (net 14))
 (segment (start 39.06 70.35) (end 39.06 46.4) (width 1) (layer F.Cu) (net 14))
 (segment (start 49.06 80.35) (end 39.06 70.35) (width 1) (layer F.Cu) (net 14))
 (segment (start 89.41 80.35) (end 49.06 80.35) (width 1) (layer F.Cu) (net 14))
 (segment (start 89.755 80.005) (end 89.41 80.35) (width 1) (layer F.Cu) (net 14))
 (segment (start 92.83 82.545) (end 48.435 82.545) (width 1) (layer F.Cu) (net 15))
 (segment (start 45.54 37.28) (end 45.54 33.07) (width 1) (layer F.Cu) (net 15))
 (segment (start 37.19 45.63) (end 45.54 37.28) (width 1) (layer F.Cu) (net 15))
 (segment (start 37.19 71.3) (end 37.19 45.63) (width 1) (layer F.Cu) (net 15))
 (segment (start 48.435 82.545) (end 37.19 71.3) (width 1) (layer F.Cu) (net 15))
 (segment (start 92.83 89.6737) (end 92.83 85.085) (width 1) (layer F.Cu) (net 16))
 (segment (start 93.98 90.8237) (end 92.83 89.6737) (width 1) (layer F.Cu) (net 16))
 (segment (start 93.98 93.09) (end 93.98 90.8237) (width 1) (layer F.Cu) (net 16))
 (segment (start 101.1973 85.8323) (end 100.45 85.085) (width 1) (layer F.Cu) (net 17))
 (segment (start 101.1973 94.114) (end 101.1973 85.8323) (width 1) (layer F.Cu) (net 17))
 (segment (start 99.955 95.3563) (end 101.1973 94.114) (width 1) (layer F.Cu) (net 17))
 (segment (start 96.52 95.3563) (end 99.955 95.3563) (width 1) (layer F.Cu) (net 17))
 (segment (start 96.52 93.09) (end 96.52 95.3563) (width 1) (layer F.Cu) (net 17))
 (segment (start 98.0497 86.5863) (end 98.0497 82.545) (width 1) (layer F.Cu) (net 18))
 (segment (start 99.06 87.5966) (end 98.0497 86.5863) (width 1) (layer F.Cu) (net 18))
 (segment (start 99.06 93.09) (end 99.06 87.5966) (width 1) (layer F.Cu) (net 18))
 (segment (start 100.45 82.545) (end 98.0497 82.545) (width 1) (layer F.Cu) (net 18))
 (segment (start 114.3487 80.005) (end 100.45 80.005) (width 1) (layer F.Cu) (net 19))
 (segment (start 114.3737 79.98) (end 114.3487 80.005) (width 1) (layer F.Cu) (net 19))
 (segment (start 116.64 79.98) (end 114.3737 79.98) (width 1) (layer F.Cu) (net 19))
 (segment (start 107.8816 77.465) (end 100.45 77.465) (width 1) (layer F.Cu) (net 20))
 (segment (start 110.4466 74.9) (end 107.8816 77.465) (width 1) (layer F.Cu) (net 20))
 (segment (start 116.64 74.9) (end 110.4466 74.9) (width 1) (layer F.Cu) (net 20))
 (segment (start 125.0752 54.85) (end 137.12 54.85) (width 1) (layer F.Cu) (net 21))
 (segment (start 105.0002 74.925) (end 125.0752 54.85) (width 1) (layer F.Cu) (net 21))
 (segment (start 100.45 74.925) (end 105.0002 74.925) (width 1) (layer F.Cu) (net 21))
 (segment (start 116.85 50.7653) (end 102.8503 64.765) (width 1) (layer F.Cu) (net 24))
 (segment (start 116.85 33.07) (end 116.85 50.7653) (width 1) (layer F.Cu) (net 24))
 (segment (start 100.45 64.765) (end 102.8503 64.765) (width 1) (layer F.Cu) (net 24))
 (segment (start 100.45 62.225) (end 102.8503 62.225) (width 1) (layer F.Cu) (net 25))
 (segment (start 114.31 50.7653) (end 102.8503 62.225) (width 1) (layer F.Cu) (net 25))
 (segment (start 114.31 33.07) (end 114.31 50.7653) (width 1) (layer F.Cu) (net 25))
 (segment (start 100.45 59.685) (end 102.8503 59.685) (width 1) (layer F.Cu) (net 26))
 (segment (start 108.63 53.9053) (end 102.8503 59.685) (width 1) (layer F.Cu) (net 26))
 (segment (start 108.63 33.13) (end 108.63 53.9053) (width 1) (layer F.Cu) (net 26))
 (segment (start 98.0497 40.5982) (end 98.0497 57.145) (width 1) (layer F.Cu) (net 27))
 (segment (start 103.1 35.5479) (end 98.0497 40.5982) (width 1) (layer F.Cu) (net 27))
 (segment (start 103.1 33.18) (end 103.1 35.5479) (width 1) (layer F.Cu) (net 27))
 (segment (start 100.45 57.145) (end 98.0497 57.145) (width 1) (layer F.Cu) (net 27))
 (segment (start 105.5201 51.9352) (end 102.8503 54.605) (width 1) (layer F.Cu) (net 28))
 (segment (start 105.5201 31.5489) (end 105.5201 51.9352) (width 1) (layer F.Cu) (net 28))
 (segment (start 104.7832 30.812) (end 105.5201 31.5489) (width 1) (layer F.Cu) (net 28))
 (segment (start 101.4395 30.812) (end 104.7832 30.812) (width 1) (layer F.Cu) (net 28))
 (segment (start 100.4979 31.7536) (end 101.4395 30.812) (width 1) (layer F.Cu) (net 28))
 (segment (start 100.4979 33.13) (end 100.4979 31.7536) (width 1) (layer F.Cu) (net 28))
 (segment (start 98.13 33.13) (end 100.4979 33.13) (width 1) (layer F.Cu) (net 28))
 (segment (start 100.45 54.605) (end 102.8503 54.605) (width 1) (layer F.Cu) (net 28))
 (segment (start 176.4937 47.31) (end 179.1137 44.69) (width 1) (layer F.Cu) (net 30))
 (segment (start 166.34 47.31) (end 176.4937 47.31) (width 1) (layer F.Cu) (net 30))
 (segment (start 181.38 44.69) (end 179.1137 44.69) (width 1) (layer F.Cu) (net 30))
 (segment (start 48.08 47.82) (end 48.08 45.47) (width 1) (layer B.Cu) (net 4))
 (segment (start 43.74 28.07) (end 48.14 28.07) (width 1) (layer B.Cu) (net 4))
 (segment (start 40.54 31.27) (end 43.74 28.07) (width 1) (layer B.Cu) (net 4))
 (segment (start 40.54 37.93) (end 40.54 31.27) (width 1) (layer B.Cu) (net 4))
 (segment (start 48.08 45.47) (end 40.54 37.93) (width 1) (layer B.Cu) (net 4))
 (segment (start 48.14 28.07) (end 48.54 28.07) (width 1) (layer F.Cu) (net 4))
 (segment (start 48.54 28.07) (end 53.25 23.36) (width 1) (layer F.Cu) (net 4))
 (segment (start 53.25 23.36) (end 134.29 23.36) (width 1) (layer F.Cu) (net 4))
 (segment (start 134.29 23.36) (end 152.19 41.26) (width 1) (layer F.Cu) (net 4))
 (segment (start 45.53 62.81) (end 48.0503 62.81) (width 1) (layer F.Cu) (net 4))
 (segment (start 48.08 60.0597) (end 49.4403 61.42) (width 1) (layer F.Cu) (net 4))
 (segment (start 48.08 47.82) (end 48.08 60.0597) (width 1) (layer F.Cu) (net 4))
 (segment (start 48.0503 62.81) (end 49.4403 61.42) (width 1) (layer F.Cu) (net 4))
 (segment (start 49.4403 61.42) (end 56.58 61.42) (width 1) (layer F.Cu) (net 4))
 (segment (start 140.93 40.14) (end 140.93 34.41) (width 0.5) (layer F.Cu) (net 5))
 (segment (start 140.93 34.41) (end 140.05 33.53) (width 0.5) (layer F.Cu) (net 5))
 (segment (start 95.04 40.6) (end 95.04 45.67) (width 1) (layer F.Cu) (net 5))
 (segment (start 132.02 27.44) (end 140.05 33.53) (width 1) (layer F.Cu) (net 5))
 (segment (start 94.59 27.53) (end 132.02 27.44) (width 1) (layer F.Cu) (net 5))
 (segment (start 91.87 28.93) (end 94.59 27.53) (width 1) (layer F.Cu) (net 5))
 (segment (start 91.87 37.43) (end 91.87 28.93) (width 1) (layer F.Cu) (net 5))
 (segment (start 95.04 40.6) (end 91.87 37.43) (width 1) (layer F.Cu) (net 5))
 (segment (start 95.2303 45.8603) (end 95.04 45.67) (width 1) (layer F.Cu) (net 5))
 (segment (start 95.2303 67.305) (end 95.2303 45.8603) (width 1) (layer F.Cu) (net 5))
 (segment (start 92.83 67.305) (end 95.2303 67.305) (width 1) (layer F.Cu) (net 5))
 (segment (start 54.5397 67.89) (end 54.6397 67.79) (width 1) (layer F.Cu) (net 5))
 (segment (start 45.53 67.89) (end 54.5397 67.89) (width 1) (layer F.Cu) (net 5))
 (segment (start 56.54 67.79) (end 56.0149 67.79) (width 1) (layer F.Cu) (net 5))
 (segment (start 56.0149 67.79) (end 54.6397 67.79) (width 1) (layer F.Cu) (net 5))
 (segment (start 90.0625 66.9378) (end 90.4297 67.305) (width 1) (layer F.Cu) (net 5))
 (segment (start 56.8671 66.9378) (end 90.0625 66.9378) (width 1) (layer F.Cu) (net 5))
 (segment (start 56.0149 67.79) (end 56.8671 66.9378) (width 1) (layer F.Cu) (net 5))
 (segment (start 92.83 67.305) (end 90.4297 67.305) (width 1) (layer F.Cu) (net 5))
 (segment (start 140.93 42.68) (end 147.06 42.68) (width 0.5) (layer F.Cu) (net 6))
 (segment (start 157.64 53.26) (end 164.39 53.26) (width 0.5) (layer F.Cu) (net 6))
 (segment (start 147.06 42.68) (end 157.64 53.26) (width 0.5) (layer F.Cu) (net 6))
 (segment (start 169.6826 52.2895) (end 169.1576 52.2895) (width 1) (layer F.Cu) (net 6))
 (segment (start 169.6826 52.2895) (end 170.2075 52.2895) (width 1) (layer F.Cu) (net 6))
 (segment (start 165.3605 52.2895) (end 164.39 53.26) (width 1) (layer F.Cu) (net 6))
 (segment (start 169.1576 52.2895) (end 165.3605 52.2895) (width 1) (layer F.Cu) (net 6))
 (segment (start 140.93 41.41) (end 138.14 41.41) (width 0.5) (layer F.Cu) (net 31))
 (segment (start 137.12 42.43) (end 137.12 47.23) (width 0.5) (layer F.Cu) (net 31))
 (segment (start 138.14 41.41) (end 137.12 42.43) (width 0.5) (layer F.Cu) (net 31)))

